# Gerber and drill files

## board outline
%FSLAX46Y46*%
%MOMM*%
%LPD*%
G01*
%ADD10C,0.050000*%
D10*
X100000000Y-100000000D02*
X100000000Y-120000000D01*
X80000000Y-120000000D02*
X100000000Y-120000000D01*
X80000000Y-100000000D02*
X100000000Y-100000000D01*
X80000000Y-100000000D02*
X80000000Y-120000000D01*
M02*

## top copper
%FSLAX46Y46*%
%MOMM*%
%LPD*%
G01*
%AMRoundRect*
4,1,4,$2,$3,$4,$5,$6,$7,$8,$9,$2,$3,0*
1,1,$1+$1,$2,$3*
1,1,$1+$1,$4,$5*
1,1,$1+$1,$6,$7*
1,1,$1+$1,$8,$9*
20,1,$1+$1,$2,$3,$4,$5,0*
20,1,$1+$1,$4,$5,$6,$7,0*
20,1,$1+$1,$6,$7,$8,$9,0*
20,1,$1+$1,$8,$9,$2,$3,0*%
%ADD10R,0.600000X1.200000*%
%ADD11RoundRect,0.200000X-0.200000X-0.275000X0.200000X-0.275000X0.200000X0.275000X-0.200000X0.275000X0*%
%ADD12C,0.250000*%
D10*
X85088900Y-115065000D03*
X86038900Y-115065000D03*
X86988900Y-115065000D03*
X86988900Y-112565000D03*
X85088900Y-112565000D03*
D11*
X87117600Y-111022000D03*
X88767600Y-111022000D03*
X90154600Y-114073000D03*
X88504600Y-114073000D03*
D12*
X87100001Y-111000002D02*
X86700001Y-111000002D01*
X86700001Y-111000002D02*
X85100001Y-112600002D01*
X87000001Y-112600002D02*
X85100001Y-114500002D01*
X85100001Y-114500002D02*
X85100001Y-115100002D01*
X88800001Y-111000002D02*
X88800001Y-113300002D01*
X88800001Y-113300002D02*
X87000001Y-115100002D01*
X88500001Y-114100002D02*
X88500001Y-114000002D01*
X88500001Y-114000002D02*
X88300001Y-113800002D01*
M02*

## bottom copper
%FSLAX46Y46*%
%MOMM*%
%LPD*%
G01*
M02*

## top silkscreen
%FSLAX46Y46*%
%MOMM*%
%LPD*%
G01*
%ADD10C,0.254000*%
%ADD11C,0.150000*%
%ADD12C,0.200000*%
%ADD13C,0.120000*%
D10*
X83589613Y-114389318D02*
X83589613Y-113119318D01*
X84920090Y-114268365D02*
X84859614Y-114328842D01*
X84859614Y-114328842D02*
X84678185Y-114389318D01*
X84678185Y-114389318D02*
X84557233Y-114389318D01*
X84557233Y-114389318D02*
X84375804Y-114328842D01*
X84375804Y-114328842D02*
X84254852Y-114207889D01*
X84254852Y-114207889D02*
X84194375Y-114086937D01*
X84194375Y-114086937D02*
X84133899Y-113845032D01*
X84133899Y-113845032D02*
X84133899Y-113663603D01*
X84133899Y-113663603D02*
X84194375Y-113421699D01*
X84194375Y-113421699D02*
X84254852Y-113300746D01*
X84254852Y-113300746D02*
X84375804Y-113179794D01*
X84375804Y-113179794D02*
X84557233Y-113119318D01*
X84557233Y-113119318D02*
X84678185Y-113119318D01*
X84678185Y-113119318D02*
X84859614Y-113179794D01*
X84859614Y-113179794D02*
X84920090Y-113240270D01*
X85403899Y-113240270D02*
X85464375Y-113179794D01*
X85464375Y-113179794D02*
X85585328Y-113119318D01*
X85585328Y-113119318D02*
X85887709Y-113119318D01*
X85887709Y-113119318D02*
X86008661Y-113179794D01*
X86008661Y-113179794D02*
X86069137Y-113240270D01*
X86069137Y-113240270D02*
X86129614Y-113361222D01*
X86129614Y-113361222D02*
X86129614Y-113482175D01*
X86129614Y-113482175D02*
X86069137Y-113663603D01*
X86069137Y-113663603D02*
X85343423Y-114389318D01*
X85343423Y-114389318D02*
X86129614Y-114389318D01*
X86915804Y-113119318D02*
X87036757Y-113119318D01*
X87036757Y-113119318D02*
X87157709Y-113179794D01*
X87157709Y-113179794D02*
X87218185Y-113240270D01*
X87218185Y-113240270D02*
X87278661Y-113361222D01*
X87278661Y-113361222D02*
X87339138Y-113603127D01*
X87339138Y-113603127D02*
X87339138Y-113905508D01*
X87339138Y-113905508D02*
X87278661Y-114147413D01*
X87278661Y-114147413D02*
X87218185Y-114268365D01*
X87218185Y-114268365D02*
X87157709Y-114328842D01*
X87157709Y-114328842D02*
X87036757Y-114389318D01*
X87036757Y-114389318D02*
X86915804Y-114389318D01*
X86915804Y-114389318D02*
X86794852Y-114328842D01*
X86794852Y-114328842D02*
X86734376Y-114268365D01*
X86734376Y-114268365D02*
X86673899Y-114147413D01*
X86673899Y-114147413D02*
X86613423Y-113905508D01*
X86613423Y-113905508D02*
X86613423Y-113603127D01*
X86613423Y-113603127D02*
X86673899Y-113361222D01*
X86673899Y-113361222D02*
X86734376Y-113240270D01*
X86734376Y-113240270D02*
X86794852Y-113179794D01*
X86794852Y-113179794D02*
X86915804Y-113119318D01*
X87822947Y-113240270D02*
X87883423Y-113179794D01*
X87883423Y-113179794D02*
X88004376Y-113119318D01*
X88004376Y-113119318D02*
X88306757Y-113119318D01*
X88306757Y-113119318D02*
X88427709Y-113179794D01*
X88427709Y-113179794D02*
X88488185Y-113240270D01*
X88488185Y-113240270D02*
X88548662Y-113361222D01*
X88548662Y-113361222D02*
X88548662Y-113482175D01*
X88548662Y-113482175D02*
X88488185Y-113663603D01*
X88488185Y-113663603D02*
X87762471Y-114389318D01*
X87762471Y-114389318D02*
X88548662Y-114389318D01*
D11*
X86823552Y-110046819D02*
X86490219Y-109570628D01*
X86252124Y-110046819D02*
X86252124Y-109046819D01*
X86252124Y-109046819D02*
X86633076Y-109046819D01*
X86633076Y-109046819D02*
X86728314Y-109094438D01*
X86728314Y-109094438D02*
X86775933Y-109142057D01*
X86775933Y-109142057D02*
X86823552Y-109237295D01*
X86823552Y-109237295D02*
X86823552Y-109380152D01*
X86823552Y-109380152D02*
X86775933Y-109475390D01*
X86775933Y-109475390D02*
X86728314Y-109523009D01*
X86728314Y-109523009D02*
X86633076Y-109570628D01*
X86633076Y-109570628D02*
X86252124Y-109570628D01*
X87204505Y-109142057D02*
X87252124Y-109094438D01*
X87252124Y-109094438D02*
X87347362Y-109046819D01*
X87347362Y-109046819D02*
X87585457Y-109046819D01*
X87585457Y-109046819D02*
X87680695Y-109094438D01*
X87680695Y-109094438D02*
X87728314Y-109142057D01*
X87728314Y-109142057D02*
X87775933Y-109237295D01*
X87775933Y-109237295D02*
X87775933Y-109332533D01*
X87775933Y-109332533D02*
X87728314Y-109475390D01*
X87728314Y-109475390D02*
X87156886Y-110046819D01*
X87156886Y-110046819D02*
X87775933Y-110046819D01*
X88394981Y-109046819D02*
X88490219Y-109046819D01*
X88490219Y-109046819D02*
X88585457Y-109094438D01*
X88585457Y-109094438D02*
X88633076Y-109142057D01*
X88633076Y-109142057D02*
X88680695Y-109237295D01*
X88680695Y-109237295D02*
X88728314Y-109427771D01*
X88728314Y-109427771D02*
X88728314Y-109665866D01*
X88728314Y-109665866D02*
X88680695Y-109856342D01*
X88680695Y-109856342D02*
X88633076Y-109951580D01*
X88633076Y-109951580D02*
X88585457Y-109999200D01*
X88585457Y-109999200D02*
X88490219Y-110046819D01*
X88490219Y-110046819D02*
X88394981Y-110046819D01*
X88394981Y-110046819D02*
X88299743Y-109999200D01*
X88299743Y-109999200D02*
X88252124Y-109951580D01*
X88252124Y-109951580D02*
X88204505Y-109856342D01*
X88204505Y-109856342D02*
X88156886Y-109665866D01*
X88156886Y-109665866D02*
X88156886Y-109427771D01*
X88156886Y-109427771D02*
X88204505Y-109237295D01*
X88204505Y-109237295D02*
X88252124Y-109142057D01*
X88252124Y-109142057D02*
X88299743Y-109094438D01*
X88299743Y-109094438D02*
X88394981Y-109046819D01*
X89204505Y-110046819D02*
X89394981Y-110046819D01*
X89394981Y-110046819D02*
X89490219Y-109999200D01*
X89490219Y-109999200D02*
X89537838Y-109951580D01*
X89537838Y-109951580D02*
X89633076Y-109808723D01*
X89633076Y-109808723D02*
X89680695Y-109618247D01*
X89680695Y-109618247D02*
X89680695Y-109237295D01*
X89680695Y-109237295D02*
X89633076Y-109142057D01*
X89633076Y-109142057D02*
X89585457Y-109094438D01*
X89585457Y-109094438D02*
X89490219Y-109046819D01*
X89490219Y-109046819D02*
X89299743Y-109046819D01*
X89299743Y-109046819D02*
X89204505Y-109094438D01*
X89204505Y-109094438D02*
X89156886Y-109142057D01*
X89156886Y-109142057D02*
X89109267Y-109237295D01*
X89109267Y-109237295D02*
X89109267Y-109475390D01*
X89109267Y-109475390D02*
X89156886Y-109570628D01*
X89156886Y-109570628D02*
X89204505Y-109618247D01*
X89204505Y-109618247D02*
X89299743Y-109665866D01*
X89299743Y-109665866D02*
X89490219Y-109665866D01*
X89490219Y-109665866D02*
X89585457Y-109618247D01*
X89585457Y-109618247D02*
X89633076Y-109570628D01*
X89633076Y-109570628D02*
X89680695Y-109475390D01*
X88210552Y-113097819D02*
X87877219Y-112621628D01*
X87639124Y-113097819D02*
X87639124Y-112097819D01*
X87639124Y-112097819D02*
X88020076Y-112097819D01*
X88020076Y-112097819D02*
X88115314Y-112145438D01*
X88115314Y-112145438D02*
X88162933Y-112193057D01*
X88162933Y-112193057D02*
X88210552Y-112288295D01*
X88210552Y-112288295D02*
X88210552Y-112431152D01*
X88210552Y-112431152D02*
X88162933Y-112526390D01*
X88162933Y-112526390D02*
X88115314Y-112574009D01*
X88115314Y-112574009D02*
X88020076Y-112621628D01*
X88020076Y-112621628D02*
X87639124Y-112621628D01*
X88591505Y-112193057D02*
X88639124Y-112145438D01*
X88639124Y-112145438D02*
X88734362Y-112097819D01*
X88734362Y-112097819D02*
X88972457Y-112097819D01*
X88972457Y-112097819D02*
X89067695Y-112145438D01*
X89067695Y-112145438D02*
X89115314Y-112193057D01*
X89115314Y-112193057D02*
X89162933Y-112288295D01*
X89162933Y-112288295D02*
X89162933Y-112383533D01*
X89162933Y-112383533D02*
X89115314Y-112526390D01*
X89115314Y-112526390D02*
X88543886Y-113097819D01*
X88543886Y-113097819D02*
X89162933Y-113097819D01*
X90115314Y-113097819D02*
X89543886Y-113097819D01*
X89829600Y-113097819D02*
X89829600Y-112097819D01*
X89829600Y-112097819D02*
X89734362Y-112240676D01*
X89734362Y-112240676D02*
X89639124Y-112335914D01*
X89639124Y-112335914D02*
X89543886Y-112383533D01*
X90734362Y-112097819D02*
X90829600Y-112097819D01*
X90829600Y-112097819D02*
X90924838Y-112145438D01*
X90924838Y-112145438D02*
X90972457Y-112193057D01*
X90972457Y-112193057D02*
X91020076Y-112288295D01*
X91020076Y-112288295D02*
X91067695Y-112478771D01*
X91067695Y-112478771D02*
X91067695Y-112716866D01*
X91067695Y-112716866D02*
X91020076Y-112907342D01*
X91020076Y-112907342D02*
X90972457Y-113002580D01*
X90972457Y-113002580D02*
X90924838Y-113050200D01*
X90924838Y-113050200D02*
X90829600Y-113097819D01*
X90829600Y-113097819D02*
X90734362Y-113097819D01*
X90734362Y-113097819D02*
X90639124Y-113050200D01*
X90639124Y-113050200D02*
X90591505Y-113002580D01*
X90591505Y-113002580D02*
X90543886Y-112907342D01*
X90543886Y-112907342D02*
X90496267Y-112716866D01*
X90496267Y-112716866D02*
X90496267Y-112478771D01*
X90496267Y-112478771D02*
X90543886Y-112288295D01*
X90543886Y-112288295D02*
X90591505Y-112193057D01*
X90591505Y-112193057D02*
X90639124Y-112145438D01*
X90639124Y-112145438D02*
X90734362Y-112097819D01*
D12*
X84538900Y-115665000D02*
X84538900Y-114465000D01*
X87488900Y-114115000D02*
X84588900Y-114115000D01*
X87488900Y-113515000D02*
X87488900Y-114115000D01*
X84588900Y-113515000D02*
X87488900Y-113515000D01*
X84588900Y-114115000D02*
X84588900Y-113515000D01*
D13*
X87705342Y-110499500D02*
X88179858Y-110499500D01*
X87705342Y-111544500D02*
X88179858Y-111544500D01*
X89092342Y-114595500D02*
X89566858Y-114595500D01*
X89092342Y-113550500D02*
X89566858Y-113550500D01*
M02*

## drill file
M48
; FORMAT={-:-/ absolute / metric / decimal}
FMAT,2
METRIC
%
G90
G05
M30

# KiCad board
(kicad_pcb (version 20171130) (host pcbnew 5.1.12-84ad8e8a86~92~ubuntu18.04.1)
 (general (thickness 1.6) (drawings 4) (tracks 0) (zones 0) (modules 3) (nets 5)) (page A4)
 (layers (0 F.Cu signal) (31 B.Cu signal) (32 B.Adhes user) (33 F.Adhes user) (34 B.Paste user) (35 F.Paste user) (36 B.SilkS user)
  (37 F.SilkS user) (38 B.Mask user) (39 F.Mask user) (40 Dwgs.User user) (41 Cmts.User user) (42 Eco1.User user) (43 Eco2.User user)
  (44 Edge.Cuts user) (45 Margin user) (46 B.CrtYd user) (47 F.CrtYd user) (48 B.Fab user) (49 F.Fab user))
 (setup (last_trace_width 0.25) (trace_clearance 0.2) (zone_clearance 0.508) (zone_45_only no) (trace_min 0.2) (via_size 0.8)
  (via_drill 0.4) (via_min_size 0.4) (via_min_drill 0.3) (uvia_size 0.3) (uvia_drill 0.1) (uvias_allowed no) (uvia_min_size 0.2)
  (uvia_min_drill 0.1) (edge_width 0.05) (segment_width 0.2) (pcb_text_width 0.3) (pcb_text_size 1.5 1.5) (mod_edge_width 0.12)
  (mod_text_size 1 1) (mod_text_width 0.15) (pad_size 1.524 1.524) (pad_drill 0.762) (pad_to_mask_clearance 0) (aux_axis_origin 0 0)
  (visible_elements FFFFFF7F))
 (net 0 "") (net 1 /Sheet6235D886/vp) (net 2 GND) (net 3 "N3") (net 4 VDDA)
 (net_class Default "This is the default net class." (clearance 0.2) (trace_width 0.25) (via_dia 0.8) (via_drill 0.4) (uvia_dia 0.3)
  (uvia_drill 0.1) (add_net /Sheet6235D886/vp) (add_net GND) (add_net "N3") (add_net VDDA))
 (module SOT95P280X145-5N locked (layer F.Cu) (at 86.038900 113.815000 90.000000)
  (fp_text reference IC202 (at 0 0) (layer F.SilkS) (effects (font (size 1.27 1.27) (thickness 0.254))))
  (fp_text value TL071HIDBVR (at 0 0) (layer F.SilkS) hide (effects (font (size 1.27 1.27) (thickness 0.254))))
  (fp_line (start -1.85 -1.5) (end -0.65 -1.5) (layer F.SilkS) (width 0.2))
  (fp_line (start -0.3 1.45) (end -0.3 -1.45) (layer F.SilkS) (width 0.2))
  (fp_line (start 0.3 1.45) (end -0.3 1.45) (layer F.SilkS) (width 0.2))
  (fp_line (start 0.3 -1.45) (end 0.3 1.45) (layer F.SilkS) (width 0.2))
  (fp_line (start -0.3 -1.45) (end 0.3 -1.45) (layer F.SilkS) (width 0.2))
  (pad 1 smd rect (at -1.25 -0.95 180.000000) (size 0.6 1.2) (layers F.Cu F.Mask F.Paste) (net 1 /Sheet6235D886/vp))
  (pad 2 smd rect (at -1.25 0 180.000000) (size 0.6 1.2) (layers F.Cu F.Mask F.Paste) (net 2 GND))
  (pad 3 smd rect (at -1.25 0.95 180.000000) (size 0.6 1.2) (layers F.Cu F.Mask F.Paste) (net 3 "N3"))
  (pad 4 smd rect (at 1.25 0.95 180.000000) (size 0.6 1.2) (layers F.Cu F.Mask F.Paste) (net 1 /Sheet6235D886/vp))
  (pad 5 smd rect (at 1.25 -0.95 180.000000) (size 0.6 1.2) (layers F.Cu F.Mask F.Paste) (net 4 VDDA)))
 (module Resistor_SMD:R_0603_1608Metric (layer F.Cu) (at 87.942600 111.022000)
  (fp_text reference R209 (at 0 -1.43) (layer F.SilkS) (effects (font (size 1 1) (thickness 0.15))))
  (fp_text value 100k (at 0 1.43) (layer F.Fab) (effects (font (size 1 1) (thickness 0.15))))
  (fp_line (start -0.237258 -0.5225) (end 0.237258 -0.5225) (layer F.SilkS) (width 0.12))
  (fp_line (start -0.237258 0.5225) (end 0.237258 0.5225) (layer F.SilkS) (width 0.12))
  (pad 1 smd roundrect (at -0.825 0) (size 0.8 0.95) (layers F.Cu F.Mask F.Paste) (roundrect_rratio 0.25) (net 4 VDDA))
  (pad 2 smd roundrect (at 0.825 0) (size 0.8 0.95) (layers F.Cu F.Mask F.Paste) (roundrect_rratio 0.25) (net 3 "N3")))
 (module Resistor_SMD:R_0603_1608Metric (layer F.Cu) (at 89.329600 114.073000)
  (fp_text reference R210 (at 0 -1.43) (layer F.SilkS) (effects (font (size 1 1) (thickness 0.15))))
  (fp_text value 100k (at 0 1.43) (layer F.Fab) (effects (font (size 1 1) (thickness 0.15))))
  (fp_line (start -0.237258 0.5225) (end 0.237258 0.5225) (layer F.SilkS) (width 0.12))
  (fp_line (start -0.237258 -0.5225) (end 0.237258 -0.5225) (layer F.SilkS) (width 0.12))
  (pad 2 smd roundrect (at 0.825 0) (size 0.8 0.95) (layers F.Cu F.Mask F.Paste) (roundrect_rratio 0.25) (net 2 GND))
  (pad 1 smd roundrect (at -0.825 0) (size 0.8 0.95) (layers F.Cu F.Mask F.Paste) (roundrect_rratio 0.25) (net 3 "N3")))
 (gr_line (start 100 100) (end 100 120) (layer Edge.Cuts) (width 0.05))
 (gr_line (start 80 120) (end 100 120) (layer Edge.Cuts) (width 0.05))
 (gr_line (start 80 100) (end 100 100) (layer Edge.Cuts) (width 0.05))
 (gr_line (start 80 100) (end 80 120) (layer Edge.Cuts) (width 0.05))
 (segment (start 87.100001 111.000002) (end 86.700001 111.000002) (width 0.250000) (layer F.Cu) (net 4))
 (segment (start 86.700001 111.000002) (end 85.100001 112.600002) (width 0.250000) (layer F.Cu) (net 4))
 (segment (start 87.000001 112.600002) (end 85.100001 114.500002) (width 0.250000) (layer F.Cu) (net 1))
 (segment (start 85.100001 114.500002) (end 85.100001 115.100002) (width 0.250000) (layer F.Cu) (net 1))
 (segment (start 88.800001 111.000002) (end 88.800001 113.300002) (width 0.250000) (layer F.Cu) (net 3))
 (segment (start 88.800001 113.300002) (end 87.000001 115.100002) (width 0.250000) (layer F.Cu) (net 3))
 (segment (start 88.500001 114.100002) (end 88.500001 114.000002) (width 0.250000) (layer F.Cu) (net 3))
 (segment (start 88.500001 114.000002) (end 88.300001 113.800002) (width 0.250000) (layer F.Cu) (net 3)))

